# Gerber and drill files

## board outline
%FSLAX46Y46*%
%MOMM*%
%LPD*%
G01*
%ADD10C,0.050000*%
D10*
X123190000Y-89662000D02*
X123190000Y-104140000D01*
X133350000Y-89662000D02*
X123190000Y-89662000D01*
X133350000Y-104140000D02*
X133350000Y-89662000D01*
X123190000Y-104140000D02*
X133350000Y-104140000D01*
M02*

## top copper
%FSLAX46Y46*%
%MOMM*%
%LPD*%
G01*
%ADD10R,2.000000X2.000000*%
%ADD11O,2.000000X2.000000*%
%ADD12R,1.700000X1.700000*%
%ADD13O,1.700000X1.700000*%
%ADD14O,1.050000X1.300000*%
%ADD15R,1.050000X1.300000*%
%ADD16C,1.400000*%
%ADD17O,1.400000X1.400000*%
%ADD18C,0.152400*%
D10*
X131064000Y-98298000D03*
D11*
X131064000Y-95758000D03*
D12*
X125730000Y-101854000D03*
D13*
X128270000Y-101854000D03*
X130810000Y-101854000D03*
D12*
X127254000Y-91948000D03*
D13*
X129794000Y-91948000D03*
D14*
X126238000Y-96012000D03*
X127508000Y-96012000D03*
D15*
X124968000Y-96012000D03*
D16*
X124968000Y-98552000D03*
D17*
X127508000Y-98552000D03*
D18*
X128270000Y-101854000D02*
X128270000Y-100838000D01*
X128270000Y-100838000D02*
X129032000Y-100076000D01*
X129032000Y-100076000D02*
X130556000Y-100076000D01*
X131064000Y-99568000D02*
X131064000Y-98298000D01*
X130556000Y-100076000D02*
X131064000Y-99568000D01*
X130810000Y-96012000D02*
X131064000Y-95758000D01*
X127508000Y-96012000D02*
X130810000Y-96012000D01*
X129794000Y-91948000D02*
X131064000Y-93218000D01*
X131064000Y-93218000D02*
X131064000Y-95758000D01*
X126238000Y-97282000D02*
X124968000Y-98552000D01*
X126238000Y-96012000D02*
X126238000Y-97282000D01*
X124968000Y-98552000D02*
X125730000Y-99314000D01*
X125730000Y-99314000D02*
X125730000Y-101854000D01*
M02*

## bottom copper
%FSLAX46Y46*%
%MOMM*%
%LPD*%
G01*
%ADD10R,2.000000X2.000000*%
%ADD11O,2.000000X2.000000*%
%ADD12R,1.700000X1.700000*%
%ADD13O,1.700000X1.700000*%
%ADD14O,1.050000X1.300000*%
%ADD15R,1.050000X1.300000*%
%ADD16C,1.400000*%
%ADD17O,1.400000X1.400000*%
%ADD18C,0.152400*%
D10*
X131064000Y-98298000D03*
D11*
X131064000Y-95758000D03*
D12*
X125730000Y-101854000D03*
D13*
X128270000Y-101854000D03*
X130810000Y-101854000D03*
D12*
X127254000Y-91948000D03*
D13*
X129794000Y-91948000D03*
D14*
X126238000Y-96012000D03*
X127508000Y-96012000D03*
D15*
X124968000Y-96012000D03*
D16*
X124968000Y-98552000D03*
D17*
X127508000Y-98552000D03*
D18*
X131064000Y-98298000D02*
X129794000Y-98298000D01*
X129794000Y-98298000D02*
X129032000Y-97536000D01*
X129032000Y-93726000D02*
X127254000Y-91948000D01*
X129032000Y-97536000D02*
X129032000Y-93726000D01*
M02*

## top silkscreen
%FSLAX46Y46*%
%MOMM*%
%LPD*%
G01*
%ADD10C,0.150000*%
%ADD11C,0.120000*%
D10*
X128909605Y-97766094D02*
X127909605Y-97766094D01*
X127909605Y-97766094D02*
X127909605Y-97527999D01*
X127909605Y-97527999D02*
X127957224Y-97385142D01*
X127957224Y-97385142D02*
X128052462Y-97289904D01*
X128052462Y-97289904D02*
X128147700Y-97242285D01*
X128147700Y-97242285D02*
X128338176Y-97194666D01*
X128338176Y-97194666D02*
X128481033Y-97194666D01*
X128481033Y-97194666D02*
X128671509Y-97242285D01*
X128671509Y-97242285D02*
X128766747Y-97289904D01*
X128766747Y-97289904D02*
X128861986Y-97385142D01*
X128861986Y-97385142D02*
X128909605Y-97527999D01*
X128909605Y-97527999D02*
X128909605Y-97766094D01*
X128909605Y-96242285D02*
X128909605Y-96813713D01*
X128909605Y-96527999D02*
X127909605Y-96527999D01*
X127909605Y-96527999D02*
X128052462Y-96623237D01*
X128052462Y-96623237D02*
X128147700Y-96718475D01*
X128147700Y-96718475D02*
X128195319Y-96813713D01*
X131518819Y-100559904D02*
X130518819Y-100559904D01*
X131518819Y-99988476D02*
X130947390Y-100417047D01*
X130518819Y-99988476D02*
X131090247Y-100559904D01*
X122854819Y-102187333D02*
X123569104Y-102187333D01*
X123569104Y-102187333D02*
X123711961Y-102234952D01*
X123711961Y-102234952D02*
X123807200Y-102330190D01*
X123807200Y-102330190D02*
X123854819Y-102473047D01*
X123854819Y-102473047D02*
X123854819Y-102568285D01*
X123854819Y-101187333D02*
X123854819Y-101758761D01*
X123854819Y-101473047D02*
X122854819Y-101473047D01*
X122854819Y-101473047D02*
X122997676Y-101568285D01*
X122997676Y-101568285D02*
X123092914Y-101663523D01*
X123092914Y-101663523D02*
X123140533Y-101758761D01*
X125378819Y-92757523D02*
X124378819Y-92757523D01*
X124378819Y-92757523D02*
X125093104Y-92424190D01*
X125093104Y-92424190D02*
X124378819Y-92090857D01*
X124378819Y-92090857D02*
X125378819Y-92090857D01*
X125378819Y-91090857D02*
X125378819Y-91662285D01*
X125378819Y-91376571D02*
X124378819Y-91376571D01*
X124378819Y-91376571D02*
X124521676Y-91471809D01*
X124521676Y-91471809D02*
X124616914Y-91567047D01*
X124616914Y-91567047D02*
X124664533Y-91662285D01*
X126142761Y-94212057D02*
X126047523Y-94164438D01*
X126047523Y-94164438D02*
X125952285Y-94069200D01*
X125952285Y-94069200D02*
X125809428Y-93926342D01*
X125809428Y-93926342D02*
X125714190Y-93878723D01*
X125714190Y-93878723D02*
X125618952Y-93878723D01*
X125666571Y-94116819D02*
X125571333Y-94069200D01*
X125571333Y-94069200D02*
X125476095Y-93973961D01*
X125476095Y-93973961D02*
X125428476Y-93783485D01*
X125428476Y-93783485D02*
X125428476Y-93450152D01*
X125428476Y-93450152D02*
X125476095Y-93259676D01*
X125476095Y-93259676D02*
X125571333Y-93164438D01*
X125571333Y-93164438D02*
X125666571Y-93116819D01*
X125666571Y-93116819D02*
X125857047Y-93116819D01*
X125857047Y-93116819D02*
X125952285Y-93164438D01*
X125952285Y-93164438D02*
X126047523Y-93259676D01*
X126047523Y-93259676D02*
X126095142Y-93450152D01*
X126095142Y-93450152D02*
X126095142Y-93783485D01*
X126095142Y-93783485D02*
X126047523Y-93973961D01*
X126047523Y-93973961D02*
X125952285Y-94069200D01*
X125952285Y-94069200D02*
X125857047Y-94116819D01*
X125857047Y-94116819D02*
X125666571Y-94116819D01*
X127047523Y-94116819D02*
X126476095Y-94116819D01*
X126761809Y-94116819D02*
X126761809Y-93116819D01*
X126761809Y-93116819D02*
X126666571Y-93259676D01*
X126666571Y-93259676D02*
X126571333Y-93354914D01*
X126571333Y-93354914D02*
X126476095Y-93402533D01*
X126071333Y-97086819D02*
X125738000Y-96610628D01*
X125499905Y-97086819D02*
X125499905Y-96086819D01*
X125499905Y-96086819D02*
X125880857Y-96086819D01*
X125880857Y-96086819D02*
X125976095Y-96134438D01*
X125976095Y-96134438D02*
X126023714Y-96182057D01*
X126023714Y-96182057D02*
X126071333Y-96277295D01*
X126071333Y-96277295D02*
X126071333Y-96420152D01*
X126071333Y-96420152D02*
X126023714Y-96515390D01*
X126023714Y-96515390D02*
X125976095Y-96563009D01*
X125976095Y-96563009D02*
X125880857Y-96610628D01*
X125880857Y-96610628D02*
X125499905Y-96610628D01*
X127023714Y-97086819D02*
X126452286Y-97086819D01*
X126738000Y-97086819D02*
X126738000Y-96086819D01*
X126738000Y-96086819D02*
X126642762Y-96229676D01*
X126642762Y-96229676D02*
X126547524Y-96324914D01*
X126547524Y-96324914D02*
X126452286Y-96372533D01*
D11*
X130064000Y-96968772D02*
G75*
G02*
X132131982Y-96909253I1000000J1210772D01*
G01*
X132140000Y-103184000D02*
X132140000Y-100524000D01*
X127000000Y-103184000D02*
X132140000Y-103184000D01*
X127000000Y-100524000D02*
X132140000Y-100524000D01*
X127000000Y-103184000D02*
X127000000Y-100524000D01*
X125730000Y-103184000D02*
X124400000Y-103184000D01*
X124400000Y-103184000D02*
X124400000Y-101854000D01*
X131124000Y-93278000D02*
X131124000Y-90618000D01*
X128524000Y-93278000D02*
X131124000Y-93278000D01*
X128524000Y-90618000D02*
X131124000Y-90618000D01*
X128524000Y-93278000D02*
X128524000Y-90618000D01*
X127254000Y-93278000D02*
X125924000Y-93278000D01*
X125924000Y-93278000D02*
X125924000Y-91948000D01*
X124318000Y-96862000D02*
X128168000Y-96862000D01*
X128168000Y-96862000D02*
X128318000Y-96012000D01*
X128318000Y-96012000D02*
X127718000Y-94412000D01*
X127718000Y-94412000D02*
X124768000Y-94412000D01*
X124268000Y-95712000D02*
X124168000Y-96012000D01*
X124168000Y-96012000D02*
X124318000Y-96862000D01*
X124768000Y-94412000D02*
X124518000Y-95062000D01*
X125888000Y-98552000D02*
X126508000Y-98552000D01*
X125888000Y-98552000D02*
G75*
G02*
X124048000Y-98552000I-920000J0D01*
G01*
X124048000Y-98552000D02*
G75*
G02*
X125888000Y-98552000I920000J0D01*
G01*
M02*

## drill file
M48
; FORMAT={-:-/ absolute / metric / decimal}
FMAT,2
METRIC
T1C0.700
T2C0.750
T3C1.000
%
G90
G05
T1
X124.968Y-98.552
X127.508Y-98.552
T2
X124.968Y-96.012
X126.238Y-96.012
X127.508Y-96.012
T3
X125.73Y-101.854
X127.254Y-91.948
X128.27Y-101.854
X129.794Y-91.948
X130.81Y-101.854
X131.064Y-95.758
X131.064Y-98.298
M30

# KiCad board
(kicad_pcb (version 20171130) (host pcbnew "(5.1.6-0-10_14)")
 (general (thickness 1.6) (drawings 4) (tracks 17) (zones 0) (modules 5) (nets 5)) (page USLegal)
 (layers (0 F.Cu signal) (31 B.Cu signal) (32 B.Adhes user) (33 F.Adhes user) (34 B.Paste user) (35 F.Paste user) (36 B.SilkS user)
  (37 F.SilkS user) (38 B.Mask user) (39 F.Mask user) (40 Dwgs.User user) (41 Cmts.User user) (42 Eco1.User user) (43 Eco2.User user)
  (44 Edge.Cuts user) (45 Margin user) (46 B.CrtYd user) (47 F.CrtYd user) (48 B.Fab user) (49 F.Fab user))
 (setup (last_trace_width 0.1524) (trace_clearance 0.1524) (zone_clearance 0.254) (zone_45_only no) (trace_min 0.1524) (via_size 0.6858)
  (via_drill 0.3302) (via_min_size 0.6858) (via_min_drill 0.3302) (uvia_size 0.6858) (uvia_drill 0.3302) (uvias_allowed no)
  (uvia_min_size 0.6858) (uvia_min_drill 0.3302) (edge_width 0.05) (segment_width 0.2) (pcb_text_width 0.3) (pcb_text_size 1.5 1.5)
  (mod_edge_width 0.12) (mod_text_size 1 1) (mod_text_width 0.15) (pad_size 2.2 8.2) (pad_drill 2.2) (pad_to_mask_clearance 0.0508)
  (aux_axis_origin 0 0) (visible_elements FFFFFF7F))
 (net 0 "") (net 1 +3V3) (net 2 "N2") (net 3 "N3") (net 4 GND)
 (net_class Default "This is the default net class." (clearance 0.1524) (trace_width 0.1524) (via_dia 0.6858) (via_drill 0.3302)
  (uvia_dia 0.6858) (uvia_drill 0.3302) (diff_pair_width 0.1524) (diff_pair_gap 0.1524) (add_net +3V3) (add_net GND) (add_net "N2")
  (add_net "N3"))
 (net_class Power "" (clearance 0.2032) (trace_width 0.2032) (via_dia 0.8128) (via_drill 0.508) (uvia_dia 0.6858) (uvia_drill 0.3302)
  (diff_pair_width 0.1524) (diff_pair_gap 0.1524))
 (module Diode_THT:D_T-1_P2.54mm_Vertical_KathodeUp (layer F.Cu) (at 131.064 98.298 90)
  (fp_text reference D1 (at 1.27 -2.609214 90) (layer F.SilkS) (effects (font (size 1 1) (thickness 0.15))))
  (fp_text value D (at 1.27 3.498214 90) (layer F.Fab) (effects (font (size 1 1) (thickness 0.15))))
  (fp_arc (start 2.54 0) (end 1.329228 -1) (angle 277.594921) (layer F.SilkS) (width 0.12))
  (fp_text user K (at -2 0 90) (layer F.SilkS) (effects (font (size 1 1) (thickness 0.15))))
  (pad 1 thru_hole rect (at 0 0 90) (size 2 2) (drill 1) (layers *.Cu *.Mask) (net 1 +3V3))
  (pad 2 thru_hole oval (at 2.54 0 90) (size 2 2) (drill 1) (layers *.Cu *.Mask) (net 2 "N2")))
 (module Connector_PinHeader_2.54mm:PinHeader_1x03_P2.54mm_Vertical (layer F.Cu) (at 125.73 101.854 90)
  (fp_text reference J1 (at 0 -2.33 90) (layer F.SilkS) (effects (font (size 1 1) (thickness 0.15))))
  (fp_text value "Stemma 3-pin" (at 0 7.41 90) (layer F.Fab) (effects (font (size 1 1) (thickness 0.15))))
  (fp_line (start -1.33 6.41) (end 1.33 6.41) (layer F.SilkS) (width 0.12))
  (fp_line (start -1.33 1.27) (end -1.33 6.41) (layer F.SilkS) (width 0.12))
  (fp_line (start 1.33 1.27) (end 1.33 6.41) (layer F.SilkS) (width 0.12))
  (fp_line (start -1.33 1.27) (end 1.33 1.27) (layer F.SilkS) (width 0.12))
  (fp_line (start -1.33 0) (end -1.33 -1.33) (layer F.SilkS) (width 0.12))
  (fp_line (start -1.33 -1.33) (end 0 -1.33) (layer F.SilkS) (width 0.12))
  (pad 1 thru_hole rect (at 0 0 90) (size 1.7 1.7) (drill 1) (layers *.Cu *.Mask) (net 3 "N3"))
  (pad 2 thru_hole oval (at 0 2.54 90) (size 1.7 1.7) (drill 1) (layers *.Cu *.Mask) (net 1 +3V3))
  (pad 3 thru_hole oval (at 0 5.08 90) (size 1.7 1.7) (drill 1) (layers *.Cu *.Mask) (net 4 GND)))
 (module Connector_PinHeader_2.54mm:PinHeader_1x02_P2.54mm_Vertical (layer F.Cu) (at 127.254 91.948 90)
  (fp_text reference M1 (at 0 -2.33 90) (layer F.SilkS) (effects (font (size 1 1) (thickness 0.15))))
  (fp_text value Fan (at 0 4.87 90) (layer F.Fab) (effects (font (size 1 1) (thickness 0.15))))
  (fp_line (start -1.33 3.87) (end 1.33 3.87) (layer F.SilkS) (width 0.12))
  (fp_line (start -1.33 1.27) (end -1.33 3.87) (layer F.SilkS) (width 0.12))
  (fp_line (start 1.33 1.27) (end 1.33 3.87) (layer F.SilkS) (width 0.12))
  (fp_line (start -1.33 1.27) (end 1.33 1.27) (layer F.SilkS) (width 0.12))
  (fp_line (start -1.33 0) (end -1.33 -1.33) (layer F.SilkS) (width 0.12))
  (fp_line (start -1.33 -1.33) (end 0 -1.33) (layer F.SilkS) (width 0.12))
  (pad 1 thru_hole rect (at 0 0 90) (size 1.7 1.7) (drill 1) (layers *.Cu *.Mask) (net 1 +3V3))
  (pad 2 thru_hole oval (at 0 2.54 90) (size 1.7 1.7) (drill 1) (layers *.Cu *.Mask) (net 2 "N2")))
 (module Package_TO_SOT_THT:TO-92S (layer F.Cu) (at 124.968 96.012)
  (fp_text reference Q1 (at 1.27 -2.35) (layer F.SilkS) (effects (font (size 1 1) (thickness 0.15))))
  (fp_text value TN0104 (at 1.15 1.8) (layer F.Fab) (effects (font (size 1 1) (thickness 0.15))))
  (fp_line (start -0.65 0.85) (end 3.2 0.85) (layer F.SilkS) (width 0.12))
  (fp_line (start 3.2 0.85) (end 3.35 0) (layer F.SilkS) (width 0.12))
  (fp_line (start 3.35 0) (end 2.75 -1.6) (layer F.SilkS) (width 0.12))
  (fp_line (start 2.75 -1.6) (end -0.2 -1.6) (layer F.SilkS) (width 0.12))
  (fp_line (start -0.7 -0.3) (end -0.8 0) (layer F.SilkS) (width 0.12))
  (fp_line (start -0.8 0) (end -0.65 0.85) (layer F.SilkS) (width 0.12))
  (fp_line (start -0.2 -1.6) (end -0.45 -0.95) (layer F.SilkS) (width 0.12))
  (pad 2 thru_hole oval (at 1.27 0 180) (size 1.05 1.3) (drill 0.75) (layers *.Cu *.Mask) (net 3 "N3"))
  (pad 3 thru_hole oval (at 2.54 0 180) (size 1.05 1.3) (drill 0.75) (layers *.Cu *.Mask) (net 2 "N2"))
  (pad 1 thru_hole rect (at 0 0 180) (size 1.05 1.3) (drill 0.75) (layers *.Cu *.Mask) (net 4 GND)))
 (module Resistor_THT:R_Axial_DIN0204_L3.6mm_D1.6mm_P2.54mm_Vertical (layer F.Cu) (at 124.968 98.552)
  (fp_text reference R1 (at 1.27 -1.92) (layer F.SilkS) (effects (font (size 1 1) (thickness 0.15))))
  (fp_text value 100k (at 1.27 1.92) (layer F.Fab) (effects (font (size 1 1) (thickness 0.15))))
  (fp_line (start 0.92 0) (end 1.54 0) (layer F.SilkS) (width 0.12))
  (fp_circle (center 0 0) (end 0.92 0) (layer F.SilkS) (width 0.12))
  (pad 1 thru_hole circle (at 0 0) (size 1.4 1.4) (drill 0.7) (layers *.Cu *.Mask) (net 3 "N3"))
  (pad 2 thru_hole oval (at 2.54 0) (size 1.4 1.4) (drill 0.7) (layers *.Cu *.Mask) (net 4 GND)))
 (gr_line (start 123.19 89.662) (end 123.19 104.14) (layer Edge.Cuts) (width 0.05))
 (gr_line (start 133.35 89.662) (end 123.19 89.662) (layer Edge.Cuts) (width 0.05))
 (gr_line (start 133.35 104.14) (end 133.35 89.662) (layer Edge.Cuts) (width 0.05))
 (gr_line (start 123.19 104.14) (end 133.35 104.14) (layer Edge.Cuts) (width 0.05))
 (segment (start 128.27 101.854) (end 128.27 100.838) (width 0.1524) (layer F.Cu) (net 1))
 (segment (start 128.27 100.838) (end 129.032 100.076) (width 0.1524) (layer F.Cu) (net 1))
 (segment (start 129.032 100.076) (end 130.556 100.076) (width 0.1524) (layer F.Cu) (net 1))
 (segment (start 131.064 99.568) (end 131.064 98.298) (width 0.1524) (layer F.Cu) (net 1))
 (segment (start 130.556 100.076) (end 131.064 99.568) (width 0.1524) (layer F.Cu) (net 1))
 (segment (start 131.064 98.298) (end 129.794 98.298) (width 0.1524) (layer B.Cu) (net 1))
 (segment (start 129.794 98.298) (end 129.032 97.536) (width 0.1524) (layer B.Cu) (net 1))
 (segment (start 129.032 93.726) (end 127.254 91.948) (width 0.1524) (layer B.Cu) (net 1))
 (segment (start 129.032 97.536) (end 129.032 93.726) (width 0.1524) (layer B.Cu) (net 1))
 (segment (start 130.81 96.012) (end 131.064 95.758) (width 0.1524) (layer F.Cu) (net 2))
 (segment (start 127.508 96.012) (end 130.81 96.012) (width 0.1524) (layer F.Cu) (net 2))
 (segment (start 129.794 91.948) (end 131.064 93.218) (width 0.1524) (layer F.Cu) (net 2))
 (segment (start 131.064 93.218) (end 131.064 95.758) (width 0.1524) (layer F.Cu) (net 2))
 (segment (start 126.238 97.282) (end 124.968 98.552) (width 0.1524) (layer F.Cu) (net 3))
 (segment (start 126.238 96.012) (end 126.238 97.282) (width 0.1524) (layer F.Cu) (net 3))
 (segment (start 124.968 98.552) (end 125.73 99.314) (width 0.1524) (layer F.Cu) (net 3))
 (segment (start 125.73 99.314) (end 125.73 101.854) (width 0.1524) (layer F.Cu) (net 3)))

